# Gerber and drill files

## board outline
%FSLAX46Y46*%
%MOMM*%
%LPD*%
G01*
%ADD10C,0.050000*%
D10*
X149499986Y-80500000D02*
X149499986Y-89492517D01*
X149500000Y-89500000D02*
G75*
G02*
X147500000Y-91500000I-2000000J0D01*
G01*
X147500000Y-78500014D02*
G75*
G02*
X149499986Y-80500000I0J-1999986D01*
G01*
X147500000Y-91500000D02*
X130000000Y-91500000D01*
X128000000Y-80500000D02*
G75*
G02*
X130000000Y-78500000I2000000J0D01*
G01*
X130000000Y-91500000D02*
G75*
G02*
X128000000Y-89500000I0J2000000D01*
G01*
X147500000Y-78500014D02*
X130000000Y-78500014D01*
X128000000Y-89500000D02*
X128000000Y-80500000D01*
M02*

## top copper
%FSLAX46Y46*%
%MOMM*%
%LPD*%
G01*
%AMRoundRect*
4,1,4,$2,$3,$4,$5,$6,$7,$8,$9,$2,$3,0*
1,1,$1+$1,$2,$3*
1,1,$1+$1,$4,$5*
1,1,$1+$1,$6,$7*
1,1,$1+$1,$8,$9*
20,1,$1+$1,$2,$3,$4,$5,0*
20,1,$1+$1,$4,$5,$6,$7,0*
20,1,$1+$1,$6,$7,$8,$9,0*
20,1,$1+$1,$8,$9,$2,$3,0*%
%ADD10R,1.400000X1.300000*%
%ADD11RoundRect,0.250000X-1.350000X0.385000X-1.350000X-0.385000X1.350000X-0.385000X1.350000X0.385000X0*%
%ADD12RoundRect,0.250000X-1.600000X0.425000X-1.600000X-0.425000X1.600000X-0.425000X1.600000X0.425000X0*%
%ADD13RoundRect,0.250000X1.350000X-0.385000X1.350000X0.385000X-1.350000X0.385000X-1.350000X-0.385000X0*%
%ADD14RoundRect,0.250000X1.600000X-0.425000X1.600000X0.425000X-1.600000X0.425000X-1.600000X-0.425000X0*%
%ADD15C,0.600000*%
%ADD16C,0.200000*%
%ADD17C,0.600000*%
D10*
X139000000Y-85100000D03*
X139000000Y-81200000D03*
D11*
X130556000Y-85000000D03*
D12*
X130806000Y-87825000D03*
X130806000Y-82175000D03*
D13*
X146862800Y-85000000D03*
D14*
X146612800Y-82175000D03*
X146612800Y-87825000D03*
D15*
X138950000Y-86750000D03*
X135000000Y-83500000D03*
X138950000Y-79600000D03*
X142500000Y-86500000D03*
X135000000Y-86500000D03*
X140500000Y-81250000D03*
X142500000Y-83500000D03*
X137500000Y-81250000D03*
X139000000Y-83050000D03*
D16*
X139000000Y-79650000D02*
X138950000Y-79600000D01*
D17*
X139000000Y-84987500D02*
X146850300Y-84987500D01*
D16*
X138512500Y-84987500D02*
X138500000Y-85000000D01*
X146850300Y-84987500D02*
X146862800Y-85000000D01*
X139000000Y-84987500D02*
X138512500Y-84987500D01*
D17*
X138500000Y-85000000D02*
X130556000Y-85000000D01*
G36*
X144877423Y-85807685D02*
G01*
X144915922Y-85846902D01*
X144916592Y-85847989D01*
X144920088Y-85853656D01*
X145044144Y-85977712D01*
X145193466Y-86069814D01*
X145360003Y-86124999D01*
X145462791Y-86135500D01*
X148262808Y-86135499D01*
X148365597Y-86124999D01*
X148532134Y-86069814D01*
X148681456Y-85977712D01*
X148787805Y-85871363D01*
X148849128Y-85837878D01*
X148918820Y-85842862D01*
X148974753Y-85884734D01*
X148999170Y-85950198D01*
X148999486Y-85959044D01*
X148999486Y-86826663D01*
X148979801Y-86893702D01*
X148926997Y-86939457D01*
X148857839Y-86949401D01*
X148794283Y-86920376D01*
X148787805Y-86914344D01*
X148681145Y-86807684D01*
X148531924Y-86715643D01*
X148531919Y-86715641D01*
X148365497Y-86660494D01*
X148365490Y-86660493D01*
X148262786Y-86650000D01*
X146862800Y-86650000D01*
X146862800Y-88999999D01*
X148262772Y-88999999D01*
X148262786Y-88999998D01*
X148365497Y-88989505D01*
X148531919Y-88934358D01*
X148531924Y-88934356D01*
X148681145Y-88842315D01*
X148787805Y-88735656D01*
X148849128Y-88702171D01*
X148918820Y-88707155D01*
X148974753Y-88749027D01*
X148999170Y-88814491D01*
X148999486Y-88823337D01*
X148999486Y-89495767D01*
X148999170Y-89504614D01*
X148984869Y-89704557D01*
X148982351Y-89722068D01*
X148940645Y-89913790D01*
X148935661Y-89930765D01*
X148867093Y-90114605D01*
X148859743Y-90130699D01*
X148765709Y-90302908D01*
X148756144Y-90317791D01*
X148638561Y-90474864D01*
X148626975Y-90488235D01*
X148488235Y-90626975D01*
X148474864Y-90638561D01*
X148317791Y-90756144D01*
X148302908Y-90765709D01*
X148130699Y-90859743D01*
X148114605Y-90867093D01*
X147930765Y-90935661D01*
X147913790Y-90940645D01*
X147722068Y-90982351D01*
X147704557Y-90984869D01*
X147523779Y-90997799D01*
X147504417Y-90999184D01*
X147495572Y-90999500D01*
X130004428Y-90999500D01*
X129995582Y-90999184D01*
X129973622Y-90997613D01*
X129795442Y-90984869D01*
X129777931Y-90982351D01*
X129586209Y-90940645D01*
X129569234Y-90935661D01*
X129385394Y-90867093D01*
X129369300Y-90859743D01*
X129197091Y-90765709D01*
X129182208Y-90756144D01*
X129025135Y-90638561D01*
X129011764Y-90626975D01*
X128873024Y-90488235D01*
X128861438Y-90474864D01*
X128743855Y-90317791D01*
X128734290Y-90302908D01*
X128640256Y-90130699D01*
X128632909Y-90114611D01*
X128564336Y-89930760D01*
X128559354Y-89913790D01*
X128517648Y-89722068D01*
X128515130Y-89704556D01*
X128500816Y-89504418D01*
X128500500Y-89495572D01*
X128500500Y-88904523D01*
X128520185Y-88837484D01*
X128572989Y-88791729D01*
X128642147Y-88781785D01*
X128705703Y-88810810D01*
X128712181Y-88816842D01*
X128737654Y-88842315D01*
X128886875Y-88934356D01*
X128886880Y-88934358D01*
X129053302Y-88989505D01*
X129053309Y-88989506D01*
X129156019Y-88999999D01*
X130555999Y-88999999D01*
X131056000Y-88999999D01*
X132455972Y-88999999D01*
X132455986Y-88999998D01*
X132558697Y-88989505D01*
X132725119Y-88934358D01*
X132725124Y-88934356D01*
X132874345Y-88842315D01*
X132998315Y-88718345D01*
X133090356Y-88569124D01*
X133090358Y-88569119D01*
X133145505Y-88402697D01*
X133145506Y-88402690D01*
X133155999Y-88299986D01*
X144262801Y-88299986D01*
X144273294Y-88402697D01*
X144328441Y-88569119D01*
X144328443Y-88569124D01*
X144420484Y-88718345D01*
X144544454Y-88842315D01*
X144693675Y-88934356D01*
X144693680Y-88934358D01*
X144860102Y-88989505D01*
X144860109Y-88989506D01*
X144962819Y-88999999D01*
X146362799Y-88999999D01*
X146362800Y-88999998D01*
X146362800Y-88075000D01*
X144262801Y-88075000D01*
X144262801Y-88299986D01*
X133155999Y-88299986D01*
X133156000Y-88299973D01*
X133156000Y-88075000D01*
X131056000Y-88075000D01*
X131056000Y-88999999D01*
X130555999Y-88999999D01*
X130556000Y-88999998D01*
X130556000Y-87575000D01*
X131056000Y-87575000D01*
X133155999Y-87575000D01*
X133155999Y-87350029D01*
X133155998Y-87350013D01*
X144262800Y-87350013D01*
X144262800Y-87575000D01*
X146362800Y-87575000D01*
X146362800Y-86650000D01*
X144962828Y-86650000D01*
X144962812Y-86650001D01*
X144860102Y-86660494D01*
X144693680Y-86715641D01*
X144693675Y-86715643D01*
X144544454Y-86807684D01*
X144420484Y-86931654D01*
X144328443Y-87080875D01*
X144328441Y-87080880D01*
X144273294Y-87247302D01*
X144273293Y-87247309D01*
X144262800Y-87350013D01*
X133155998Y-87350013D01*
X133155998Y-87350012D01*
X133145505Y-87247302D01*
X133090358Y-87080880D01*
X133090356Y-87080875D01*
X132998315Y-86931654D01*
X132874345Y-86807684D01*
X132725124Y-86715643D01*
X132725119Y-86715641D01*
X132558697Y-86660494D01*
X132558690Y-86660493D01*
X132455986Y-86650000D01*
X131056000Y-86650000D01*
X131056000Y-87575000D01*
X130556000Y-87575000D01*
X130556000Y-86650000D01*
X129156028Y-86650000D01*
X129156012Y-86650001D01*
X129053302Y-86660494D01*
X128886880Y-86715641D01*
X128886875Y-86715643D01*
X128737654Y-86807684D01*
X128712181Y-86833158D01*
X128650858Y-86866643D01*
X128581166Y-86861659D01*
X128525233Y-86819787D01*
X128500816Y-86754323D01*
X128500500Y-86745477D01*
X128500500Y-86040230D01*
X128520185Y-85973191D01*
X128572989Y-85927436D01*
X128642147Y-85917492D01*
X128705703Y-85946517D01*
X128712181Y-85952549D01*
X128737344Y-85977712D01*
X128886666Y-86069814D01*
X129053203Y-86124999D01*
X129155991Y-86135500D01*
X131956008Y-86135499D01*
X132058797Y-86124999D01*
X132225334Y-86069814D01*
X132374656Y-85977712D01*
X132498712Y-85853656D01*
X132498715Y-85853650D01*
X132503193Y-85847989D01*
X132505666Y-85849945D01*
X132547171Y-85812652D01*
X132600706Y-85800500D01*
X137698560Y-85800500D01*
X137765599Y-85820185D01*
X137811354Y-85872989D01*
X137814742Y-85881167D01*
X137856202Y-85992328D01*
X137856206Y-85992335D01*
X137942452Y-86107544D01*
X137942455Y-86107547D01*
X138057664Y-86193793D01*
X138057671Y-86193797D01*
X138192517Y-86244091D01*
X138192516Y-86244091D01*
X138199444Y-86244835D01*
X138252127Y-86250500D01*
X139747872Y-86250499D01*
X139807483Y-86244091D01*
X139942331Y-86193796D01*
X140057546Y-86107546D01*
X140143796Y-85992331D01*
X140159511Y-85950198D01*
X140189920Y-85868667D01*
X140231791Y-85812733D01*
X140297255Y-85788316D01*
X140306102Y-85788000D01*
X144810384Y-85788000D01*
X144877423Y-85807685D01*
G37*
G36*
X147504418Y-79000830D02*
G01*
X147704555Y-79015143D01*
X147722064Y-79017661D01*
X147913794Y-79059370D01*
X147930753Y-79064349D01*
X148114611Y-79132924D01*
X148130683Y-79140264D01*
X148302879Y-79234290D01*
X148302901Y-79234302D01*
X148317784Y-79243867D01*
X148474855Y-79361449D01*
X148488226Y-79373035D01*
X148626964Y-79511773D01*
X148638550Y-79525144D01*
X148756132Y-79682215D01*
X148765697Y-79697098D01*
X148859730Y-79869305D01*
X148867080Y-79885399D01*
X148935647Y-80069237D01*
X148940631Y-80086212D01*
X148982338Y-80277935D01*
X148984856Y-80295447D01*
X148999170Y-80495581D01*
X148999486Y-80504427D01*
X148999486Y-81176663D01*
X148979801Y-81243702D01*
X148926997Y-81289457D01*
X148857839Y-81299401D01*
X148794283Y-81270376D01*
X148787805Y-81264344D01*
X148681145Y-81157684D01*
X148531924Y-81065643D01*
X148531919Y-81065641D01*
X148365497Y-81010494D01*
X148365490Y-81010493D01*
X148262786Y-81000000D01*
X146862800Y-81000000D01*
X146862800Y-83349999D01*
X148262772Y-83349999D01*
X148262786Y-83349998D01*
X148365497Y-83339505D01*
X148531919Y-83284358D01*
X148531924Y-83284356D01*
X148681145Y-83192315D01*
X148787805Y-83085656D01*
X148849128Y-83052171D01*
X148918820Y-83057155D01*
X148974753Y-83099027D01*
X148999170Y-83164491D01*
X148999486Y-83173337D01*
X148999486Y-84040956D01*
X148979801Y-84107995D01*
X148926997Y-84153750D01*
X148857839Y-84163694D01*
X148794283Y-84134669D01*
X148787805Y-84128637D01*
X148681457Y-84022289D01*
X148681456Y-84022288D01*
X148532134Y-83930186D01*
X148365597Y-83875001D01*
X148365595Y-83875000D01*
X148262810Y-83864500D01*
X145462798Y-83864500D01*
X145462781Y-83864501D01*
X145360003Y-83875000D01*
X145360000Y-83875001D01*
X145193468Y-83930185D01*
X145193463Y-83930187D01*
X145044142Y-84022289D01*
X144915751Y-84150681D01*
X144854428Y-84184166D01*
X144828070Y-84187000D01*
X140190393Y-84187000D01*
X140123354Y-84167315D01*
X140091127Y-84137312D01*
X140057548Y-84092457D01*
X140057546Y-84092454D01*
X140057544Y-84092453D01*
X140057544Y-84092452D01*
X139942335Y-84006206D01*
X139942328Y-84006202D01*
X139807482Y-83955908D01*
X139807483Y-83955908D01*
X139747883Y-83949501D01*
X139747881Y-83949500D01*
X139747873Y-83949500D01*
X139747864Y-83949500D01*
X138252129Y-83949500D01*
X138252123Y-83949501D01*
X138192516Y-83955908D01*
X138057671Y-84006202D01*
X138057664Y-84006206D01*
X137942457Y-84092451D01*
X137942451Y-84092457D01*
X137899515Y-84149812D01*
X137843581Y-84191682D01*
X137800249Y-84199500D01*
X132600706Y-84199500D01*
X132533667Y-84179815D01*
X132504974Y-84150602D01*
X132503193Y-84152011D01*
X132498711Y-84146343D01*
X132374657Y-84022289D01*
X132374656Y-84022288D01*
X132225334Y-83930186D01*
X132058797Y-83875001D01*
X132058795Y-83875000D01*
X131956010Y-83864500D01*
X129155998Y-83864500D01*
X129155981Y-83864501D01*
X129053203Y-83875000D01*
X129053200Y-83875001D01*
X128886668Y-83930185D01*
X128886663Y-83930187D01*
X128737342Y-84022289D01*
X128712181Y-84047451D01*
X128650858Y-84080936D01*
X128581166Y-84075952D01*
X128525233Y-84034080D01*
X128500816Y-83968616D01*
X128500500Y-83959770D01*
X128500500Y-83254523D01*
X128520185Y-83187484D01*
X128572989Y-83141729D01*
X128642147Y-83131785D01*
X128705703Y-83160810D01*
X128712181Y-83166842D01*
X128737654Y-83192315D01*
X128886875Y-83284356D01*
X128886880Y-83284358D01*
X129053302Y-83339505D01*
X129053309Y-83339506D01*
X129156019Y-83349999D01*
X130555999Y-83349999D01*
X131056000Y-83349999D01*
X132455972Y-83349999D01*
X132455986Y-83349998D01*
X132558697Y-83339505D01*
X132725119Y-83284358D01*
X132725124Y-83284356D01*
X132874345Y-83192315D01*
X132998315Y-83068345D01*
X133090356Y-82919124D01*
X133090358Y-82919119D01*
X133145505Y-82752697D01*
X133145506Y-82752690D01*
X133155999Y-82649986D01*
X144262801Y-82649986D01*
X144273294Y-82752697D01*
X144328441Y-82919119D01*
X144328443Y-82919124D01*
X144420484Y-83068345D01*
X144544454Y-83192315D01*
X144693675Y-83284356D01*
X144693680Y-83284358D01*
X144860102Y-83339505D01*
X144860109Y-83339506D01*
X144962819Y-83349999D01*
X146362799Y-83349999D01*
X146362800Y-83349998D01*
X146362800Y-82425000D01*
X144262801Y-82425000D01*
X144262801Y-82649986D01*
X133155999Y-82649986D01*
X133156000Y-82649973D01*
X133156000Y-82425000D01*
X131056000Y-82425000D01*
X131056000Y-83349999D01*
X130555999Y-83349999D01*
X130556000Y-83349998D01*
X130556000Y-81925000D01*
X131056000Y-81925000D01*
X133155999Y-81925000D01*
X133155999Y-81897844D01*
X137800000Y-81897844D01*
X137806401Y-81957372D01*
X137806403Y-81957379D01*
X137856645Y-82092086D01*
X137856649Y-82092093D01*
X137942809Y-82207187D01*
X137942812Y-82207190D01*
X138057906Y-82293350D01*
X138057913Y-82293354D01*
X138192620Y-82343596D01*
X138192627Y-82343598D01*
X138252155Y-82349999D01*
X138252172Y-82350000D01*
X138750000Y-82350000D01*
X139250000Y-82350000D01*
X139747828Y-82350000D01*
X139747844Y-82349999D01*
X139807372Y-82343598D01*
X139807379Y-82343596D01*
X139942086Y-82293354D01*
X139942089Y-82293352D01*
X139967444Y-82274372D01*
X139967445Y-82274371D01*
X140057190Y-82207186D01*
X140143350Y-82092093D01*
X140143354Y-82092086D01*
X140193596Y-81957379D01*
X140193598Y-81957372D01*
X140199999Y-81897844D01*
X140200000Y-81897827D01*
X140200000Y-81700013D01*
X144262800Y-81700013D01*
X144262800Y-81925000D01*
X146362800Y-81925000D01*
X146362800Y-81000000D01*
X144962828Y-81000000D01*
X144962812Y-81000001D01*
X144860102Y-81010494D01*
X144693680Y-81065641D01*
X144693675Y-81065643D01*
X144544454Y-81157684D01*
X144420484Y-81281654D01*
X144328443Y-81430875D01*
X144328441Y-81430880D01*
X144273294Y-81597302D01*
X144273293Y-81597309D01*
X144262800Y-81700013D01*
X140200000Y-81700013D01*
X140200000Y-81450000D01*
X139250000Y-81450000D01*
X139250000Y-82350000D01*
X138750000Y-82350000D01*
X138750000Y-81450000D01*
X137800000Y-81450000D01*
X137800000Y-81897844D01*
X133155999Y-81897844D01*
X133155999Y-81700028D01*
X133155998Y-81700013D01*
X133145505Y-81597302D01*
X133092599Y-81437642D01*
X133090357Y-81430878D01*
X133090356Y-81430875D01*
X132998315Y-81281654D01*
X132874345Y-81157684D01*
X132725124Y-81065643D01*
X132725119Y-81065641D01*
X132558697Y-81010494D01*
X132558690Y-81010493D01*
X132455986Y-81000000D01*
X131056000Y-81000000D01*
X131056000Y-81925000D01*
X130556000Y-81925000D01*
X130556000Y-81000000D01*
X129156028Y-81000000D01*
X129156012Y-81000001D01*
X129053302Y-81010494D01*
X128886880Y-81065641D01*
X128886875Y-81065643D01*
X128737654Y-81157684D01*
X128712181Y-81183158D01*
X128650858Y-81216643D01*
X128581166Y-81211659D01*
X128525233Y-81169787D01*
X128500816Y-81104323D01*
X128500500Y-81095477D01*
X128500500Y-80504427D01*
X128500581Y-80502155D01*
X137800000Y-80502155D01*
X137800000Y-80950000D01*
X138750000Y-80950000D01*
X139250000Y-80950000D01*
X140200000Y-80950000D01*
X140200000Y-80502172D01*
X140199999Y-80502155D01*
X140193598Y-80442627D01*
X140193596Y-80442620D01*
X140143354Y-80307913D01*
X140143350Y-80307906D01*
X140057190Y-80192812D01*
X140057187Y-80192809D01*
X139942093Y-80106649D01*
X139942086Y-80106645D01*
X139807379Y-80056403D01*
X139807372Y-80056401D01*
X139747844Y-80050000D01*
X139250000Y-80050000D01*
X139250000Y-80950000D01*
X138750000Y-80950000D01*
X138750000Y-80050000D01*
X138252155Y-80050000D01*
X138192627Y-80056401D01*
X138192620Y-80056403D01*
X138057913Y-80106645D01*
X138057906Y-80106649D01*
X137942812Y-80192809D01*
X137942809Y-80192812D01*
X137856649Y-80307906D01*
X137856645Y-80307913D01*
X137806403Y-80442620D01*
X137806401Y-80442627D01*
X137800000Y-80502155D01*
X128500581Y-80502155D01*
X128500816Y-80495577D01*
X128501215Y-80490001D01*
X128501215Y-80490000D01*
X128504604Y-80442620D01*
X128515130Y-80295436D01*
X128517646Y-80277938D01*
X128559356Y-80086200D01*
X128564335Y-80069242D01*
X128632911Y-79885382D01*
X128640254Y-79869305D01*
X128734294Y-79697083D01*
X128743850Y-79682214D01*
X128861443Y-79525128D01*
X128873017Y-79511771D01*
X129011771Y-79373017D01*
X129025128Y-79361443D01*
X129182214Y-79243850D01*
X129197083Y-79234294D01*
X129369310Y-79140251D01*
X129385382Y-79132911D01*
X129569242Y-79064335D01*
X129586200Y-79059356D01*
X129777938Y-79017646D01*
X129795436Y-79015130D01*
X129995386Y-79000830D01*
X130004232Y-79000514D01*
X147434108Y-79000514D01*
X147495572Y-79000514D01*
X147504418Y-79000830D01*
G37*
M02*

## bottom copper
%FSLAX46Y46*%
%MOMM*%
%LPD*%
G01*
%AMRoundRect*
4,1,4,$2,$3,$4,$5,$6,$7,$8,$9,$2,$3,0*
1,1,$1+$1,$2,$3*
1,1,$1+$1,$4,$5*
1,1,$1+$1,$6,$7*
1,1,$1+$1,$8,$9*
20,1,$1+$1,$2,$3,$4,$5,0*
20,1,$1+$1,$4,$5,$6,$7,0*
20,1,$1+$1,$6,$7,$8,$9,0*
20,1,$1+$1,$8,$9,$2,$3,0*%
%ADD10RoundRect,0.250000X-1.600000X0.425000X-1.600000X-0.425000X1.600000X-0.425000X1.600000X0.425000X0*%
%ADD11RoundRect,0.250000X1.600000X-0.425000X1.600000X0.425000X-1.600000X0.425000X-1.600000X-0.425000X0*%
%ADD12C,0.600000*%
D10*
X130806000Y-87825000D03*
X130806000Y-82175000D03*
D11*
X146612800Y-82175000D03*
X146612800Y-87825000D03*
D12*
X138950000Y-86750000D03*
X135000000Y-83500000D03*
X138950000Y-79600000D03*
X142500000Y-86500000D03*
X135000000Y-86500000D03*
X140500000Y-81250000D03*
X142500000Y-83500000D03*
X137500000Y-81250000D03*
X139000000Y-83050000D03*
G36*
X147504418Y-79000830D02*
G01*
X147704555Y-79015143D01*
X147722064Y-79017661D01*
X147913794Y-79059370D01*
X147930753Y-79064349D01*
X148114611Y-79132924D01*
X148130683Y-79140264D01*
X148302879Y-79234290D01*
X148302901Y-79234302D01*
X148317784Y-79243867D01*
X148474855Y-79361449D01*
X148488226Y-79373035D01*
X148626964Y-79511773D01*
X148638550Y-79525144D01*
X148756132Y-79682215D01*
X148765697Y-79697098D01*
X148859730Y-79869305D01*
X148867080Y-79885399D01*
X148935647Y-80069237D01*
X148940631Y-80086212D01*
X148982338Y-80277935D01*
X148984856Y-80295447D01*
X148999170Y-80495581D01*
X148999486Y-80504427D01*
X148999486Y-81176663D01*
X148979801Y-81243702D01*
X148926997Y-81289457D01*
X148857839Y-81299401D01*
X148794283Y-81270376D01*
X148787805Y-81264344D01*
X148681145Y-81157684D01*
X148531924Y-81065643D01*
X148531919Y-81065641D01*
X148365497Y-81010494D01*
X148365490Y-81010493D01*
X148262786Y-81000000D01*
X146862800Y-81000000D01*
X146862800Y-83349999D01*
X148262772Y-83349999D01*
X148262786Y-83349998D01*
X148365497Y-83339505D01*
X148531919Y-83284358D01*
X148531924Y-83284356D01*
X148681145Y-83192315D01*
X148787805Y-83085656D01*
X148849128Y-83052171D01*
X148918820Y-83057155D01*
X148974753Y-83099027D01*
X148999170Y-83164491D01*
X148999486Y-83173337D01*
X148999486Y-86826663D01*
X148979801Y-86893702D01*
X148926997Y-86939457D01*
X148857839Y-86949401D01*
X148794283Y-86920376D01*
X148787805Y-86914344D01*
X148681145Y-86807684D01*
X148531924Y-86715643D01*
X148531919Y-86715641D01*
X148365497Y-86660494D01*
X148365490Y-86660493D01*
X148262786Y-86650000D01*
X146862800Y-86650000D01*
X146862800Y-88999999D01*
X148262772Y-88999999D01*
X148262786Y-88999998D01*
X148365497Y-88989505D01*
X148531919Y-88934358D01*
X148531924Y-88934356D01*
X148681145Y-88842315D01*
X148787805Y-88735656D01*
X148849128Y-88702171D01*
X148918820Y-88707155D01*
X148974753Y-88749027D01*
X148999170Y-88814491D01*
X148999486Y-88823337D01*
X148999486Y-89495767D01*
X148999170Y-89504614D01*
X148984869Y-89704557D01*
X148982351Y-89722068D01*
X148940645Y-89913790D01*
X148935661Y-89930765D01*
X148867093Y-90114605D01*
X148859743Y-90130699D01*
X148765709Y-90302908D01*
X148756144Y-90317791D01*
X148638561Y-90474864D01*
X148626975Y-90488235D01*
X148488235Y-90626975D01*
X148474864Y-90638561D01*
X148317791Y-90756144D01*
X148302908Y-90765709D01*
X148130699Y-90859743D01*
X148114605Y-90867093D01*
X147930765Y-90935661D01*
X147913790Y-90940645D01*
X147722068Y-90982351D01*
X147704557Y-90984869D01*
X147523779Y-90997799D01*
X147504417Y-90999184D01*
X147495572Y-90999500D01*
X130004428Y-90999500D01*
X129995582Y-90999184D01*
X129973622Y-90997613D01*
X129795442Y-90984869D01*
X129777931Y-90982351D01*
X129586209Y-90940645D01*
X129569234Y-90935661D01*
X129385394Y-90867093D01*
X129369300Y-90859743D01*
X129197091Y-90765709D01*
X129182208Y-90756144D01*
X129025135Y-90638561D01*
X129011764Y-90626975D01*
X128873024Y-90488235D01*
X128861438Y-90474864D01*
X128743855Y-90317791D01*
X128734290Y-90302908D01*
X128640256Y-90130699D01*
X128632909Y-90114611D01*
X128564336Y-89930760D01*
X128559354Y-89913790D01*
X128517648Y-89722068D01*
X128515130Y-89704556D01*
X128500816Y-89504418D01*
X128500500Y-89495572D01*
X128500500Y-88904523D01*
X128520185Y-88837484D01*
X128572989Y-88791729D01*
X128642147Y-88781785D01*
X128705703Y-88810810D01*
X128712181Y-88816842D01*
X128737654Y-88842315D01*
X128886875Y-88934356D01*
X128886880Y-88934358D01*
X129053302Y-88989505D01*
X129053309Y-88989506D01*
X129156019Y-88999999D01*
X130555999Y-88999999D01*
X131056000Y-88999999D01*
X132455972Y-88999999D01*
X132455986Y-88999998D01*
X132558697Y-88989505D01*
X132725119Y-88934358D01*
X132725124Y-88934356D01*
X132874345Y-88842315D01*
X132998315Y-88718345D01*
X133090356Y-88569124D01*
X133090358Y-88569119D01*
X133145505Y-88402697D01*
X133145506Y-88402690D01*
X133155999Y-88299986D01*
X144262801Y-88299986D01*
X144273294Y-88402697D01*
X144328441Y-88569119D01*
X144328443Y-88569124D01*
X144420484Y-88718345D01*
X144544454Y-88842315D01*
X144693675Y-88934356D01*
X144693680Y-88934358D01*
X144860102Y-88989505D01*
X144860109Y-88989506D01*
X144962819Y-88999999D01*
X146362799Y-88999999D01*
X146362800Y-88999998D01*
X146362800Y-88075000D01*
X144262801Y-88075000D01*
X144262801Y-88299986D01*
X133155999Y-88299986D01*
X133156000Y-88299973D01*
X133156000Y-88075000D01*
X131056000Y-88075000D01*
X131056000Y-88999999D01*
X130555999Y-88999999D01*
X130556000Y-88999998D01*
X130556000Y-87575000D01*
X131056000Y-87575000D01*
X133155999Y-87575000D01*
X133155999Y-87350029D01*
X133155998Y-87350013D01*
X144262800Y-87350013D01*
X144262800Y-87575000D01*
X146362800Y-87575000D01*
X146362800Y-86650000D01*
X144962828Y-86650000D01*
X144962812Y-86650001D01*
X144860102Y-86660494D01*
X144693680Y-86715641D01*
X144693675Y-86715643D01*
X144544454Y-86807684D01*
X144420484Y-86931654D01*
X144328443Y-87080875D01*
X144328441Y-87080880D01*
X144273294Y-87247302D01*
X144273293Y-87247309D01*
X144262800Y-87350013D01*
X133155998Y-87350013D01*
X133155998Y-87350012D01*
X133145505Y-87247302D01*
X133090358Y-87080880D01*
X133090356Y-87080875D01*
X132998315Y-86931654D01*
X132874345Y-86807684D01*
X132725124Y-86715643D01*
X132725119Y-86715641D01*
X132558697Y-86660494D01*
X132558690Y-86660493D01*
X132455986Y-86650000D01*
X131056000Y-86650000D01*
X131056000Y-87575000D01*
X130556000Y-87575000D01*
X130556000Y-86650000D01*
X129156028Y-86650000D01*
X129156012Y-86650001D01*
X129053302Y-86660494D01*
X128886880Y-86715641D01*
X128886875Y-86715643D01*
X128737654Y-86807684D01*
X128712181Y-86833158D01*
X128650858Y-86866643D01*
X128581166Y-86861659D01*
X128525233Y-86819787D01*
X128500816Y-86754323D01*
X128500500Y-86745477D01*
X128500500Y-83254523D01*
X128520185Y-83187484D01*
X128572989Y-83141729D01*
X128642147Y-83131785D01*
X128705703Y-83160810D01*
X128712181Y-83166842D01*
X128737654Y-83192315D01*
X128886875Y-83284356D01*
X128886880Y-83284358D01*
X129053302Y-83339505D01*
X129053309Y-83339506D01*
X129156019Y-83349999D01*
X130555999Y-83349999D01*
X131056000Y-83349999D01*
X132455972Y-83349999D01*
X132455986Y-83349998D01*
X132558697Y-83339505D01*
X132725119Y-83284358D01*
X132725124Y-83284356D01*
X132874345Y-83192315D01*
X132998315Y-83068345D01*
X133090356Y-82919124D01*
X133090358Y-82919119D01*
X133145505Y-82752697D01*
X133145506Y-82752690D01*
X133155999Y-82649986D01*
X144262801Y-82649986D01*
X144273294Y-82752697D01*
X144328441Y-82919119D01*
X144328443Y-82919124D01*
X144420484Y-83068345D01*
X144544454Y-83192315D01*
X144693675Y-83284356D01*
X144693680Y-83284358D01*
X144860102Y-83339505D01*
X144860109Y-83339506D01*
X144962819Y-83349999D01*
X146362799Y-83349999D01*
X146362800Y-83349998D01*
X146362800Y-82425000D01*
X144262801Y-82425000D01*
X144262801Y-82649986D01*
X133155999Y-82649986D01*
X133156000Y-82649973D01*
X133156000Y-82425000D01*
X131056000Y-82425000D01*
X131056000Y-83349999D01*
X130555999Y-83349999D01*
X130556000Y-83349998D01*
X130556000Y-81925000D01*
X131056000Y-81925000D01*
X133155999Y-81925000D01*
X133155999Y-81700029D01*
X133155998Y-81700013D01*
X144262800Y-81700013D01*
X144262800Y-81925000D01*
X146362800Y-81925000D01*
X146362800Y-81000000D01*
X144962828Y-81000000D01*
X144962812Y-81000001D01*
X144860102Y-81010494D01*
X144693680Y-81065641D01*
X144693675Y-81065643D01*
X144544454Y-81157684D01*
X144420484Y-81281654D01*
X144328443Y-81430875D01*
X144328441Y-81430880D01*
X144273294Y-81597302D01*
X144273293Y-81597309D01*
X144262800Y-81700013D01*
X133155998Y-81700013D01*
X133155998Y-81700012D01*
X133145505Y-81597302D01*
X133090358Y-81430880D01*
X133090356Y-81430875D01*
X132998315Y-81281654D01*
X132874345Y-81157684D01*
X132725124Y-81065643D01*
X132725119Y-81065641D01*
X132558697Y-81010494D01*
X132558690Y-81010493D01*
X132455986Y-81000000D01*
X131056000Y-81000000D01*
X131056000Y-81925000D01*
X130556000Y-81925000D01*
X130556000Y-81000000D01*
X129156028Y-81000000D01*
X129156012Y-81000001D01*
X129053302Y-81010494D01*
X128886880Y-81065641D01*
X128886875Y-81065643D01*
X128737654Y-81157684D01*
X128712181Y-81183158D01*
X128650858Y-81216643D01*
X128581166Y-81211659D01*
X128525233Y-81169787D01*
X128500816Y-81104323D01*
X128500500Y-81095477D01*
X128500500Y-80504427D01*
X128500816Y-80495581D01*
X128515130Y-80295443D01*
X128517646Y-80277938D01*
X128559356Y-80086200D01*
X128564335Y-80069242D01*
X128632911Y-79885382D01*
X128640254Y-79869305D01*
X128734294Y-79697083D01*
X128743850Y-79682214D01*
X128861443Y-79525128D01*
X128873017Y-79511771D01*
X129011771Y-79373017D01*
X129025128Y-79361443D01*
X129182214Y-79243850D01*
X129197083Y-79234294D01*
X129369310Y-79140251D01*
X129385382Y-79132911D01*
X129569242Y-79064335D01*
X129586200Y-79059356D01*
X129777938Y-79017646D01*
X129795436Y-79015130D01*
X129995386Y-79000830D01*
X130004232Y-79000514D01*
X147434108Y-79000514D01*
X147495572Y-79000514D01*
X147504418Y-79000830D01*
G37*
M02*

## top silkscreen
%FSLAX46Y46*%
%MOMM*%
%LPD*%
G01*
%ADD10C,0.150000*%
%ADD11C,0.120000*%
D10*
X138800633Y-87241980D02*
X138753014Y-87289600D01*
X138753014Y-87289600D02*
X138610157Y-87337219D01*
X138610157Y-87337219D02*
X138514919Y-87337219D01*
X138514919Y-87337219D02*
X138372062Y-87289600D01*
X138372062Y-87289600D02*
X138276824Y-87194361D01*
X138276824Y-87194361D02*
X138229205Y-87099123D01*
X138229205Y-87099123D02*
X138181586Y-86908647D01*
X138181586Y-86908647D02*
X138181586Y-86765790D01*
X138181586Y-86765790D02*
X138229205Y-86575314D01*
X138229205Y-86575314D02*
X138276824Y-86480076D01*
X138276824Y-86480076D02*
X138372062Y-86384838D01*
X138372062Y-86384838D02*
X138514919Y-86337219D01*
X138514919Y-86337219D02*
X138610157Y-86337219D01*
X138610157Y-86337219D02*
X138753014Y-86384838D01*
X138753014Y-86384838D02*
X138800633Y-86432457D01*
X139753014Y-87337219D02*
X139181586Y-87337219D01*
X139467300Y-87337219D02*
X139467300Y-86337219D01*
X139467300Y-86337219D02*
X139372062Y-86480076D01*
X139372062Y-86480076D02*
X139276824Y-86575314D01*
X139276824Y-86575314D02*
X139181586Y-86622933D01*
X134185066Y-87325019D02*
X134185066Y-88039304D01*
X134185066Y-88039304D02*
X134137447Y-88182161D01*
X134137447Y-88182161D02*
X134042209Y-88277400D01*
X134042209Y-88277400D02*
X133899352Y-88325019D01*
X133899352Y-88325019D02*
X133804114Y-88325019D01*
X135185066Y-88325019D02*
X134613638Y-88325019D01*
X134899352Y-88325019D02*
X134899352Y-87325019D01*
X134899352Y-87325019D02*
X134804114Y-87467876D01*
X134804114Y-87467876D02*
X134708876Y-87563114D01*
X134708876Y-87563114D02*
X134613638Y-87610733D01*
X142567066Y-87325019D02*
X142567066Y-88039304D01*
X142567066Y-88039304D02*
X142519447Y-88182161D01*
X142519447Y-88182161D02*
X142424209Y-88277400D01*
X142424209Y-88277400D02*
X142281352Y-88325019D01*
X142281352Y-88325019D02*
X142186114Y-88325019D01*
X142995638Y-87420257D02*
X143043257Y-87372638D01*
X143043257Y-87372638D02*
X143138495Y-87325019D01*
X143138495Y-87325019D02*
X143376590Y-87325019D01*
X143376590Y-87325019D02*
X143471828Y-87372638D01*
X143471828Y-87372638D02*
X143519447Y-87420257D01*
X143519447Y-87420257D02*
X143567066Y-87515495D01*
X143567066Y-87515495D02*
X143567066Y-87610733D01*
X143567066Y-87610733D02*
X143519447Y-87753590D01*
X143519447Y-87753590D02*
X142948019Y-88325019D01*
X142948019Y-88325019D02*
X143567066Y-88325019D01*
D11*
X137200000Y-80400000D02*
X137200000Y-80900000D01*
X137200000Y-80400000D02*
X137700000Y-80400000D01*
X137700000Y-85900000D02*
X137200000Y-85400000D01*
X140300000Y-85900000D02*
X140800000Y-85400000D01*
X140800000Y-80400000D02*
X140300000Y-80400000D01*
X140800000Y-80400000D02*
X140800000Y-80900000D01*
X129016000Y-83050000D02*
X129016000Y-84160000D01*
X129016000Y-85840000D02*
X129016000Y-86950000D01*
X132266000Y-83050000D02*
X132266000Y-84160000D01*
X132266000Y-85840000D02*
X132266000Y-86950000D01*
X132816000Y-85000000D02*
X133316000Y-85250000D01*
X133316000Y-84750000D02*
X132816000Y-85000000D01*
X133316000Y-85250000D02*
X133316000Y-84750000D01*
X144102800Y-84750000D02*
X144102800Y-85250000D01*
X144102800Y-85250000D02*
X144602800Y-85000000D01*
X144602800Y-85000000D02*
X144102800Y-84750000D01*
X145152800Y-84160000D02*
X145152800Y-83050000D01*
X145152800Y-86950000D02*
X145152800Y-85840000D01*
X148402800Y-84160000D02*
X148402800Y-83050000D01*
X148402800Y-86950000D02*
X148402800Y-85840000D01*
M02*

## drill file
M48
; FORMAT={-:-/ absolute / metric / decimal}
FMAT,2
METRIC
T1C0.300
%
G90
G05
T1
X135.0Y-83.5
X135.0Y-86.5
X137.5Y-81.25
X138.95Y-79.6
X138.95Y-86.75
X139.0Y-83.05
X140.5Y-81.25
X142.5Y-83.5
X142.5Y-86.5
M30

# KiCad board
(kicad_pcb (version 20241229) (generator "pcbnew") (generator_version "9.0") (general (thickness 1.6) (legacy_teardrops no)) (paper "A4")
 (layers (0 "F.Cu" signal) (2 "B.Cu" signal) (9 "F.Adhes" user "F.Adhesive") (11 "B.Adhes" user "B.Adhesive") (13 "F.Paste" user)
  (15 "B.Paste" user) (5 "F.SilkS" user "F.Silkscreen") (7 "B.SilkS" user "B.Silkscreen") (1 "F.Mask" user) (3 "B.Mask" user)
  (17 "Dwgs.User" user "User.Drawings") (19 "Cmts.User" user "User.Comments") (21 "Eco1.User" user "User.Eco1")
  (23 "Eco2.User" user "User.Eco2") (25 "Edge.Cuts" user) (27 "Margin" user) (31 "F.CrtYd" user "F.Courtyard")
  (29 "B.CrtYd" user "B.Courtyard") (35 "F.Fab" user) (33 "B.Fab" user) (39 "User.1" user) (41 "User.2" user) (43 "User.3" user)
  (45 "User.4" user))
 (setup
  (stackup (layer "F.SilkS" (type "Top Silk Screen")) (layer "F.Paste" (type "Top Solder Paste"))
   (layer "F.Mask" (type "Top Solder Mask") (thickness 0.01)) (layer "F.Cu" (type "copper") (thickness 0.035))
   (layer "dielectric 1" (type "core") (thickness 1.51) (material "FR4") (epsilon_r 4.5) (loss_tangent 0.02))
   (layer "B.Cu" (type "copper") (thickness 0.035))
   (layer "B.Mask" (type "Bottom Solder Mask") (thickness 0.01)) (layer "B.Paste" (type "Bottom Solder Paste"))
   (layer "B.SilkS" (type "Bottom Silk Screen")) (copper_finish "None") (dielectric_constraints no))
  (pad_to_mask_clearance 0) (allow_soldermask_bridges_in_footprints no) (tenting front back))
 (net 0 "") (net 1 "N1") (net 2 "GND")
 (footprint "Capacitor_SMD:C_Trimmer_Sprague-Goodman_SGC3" (layer "F.Cu") (at 139 83.15 90)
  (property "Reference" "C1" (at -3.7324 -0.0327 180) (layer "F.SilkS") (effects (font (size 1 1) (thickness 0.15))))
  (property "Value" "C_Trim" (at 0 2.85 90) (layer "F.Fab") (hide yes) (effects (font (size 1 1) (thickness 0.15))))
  (fp_line (start 2.75 -1.8) (end 2.25 -1.8) (stroke (width 0.12) (type solid)) (layer "F.SilkS"))
  (fp_line (start 2.75 -1.8) (end 2.75 -1.3) (stroke (width 0.12) (type solid)) (layer "F.SilkS"))
  (fp_line (start -2.75 -1.3) (end -2.25 -1.8) (stroke (width 0.12) (type solid)) (layer "F.SilkS"))
  (fp_line (start -2.75 1.3) (end -2.25 1.8) (stroke (width 0.12) (type solid)) (layer "F.SilkS"))
  (fp_line (start 2.75 1.8) (end 2.75 1.3) (stroke (width 0.12) (type solid)) (layer "F.SilkS"))
  (fp_line (start 2.75 1.8) (end 2.25 1.8) (stroke (width 0.12) (type solid)) (layer "F.SilkS"))
  (pad "1" smd rect (at -1.95 0 90) (size 1.3 1.4) (layers "F.Cu" "F.Mask" "F.Paste") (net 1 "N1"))
  (pad "2" smd rect (at 1.95 0 90) (size 1.3 1.4) (layers "F.Cu" "F.Mask" "F.Paste") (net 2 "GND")))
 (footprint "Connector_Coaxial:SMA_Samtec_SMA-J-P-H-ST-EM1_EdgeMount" (layer "F.Cu") (at 130.556 85 180)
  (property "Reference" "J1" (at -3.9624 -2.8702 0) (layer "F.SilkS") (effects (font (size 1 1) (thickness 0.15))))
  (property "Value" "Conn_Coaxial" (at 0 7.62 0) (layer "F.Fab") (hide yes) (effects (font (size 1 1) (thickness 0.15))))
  (fp_line (start 1.54 1.95) (end 1.54 0.84) (stroke (width 0.12) (type solid)) (layer "F.SilkS"))
  (fp_line (start 1.54 -0.84) (end 1.54 -1.95) (stroke (width 0.12) (type solid)) (layer "F.SilkS"))
  (fp_line (start -1.71 1.95) (end -1.71 0.84) (stroke (width 0.12) (type solid)) (layer "F.SilkS"))
  (fp_line (start -1.71 -0.84) (end -1.71 -1.95) (stroke (width 0.12) (type solid)) (layer "F.SilkS"))
  (fp_line (start -2.26 0) (end -2.76 -0.25) (stroke (width 0.12) (type solid)) (layer "F.SilkS"))
  (fp_line (start -2.76 0.25) (end -2.26 0) (stroke (width 0.12) (type solid)) (layer "F.SilkS"))
  (fp_line (start -2.76 -0.25) (end -2.76 0.25) (stroke (width 0.12) (type solid)) (layer "F.SilkS"))
  (pad "1" smd roundrect (at 0 0 270) (size 1.27 3.2) (layers "F.Cu" "F.Mask") (roundrect_rratio 0.1968503937) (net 1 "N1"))
  (pad "2" smd roundrect (at -0.25 -2.825 270) (size 1.35 3.7) (layers "F.Cu" "F.Mask") (roundrect_rratio 0.1851851852) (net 2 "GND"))
  (pad "2" smd roundrect (at -0.25 -2.825 270) (size 1.35 3.7) (layers "B.Cu" "B.Mask") (roundrect_rratio 0.1851851852) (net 2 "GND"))
  (pad "2" smd roundrect (at -0.25 2.825 270) (size 1.35 3.7) (layers "F.Cu" "F.Mask") (roundrect_rratio 0.1851851852) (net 2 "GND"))
  (pad "2" smd roundrect (at -0.25 2.825 270) (size 1.35 3.7) (layers "B.Cu" "B.Mask") (roundrect_rratio 0.1851851852) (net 2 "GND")))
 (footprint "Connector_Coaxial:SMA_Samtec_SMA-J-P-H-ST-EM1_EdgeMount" (layer "F.Cu") (at 146.8628 85)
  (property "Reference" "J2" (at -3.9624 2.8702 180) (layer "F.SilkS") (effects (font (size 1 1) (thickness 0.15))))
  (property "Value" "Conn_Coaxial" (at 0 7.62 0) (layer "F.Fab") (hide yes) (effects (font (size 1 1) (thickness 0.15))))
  (fp_line (start -2.76 -0.25) (end -2.76 0.25) (stroke (width 0.12) (type solid)) (layer "F.SilkS"))
  (fp_line (start -2.76 0.25) (end -2.26 0) (stroke (width 0.12) (type solid)) (layer "F.SilkS"))
  (fp_line (start -2.26 0) (end -2.76 -0.25) (stroke (width 0.12) (type solid)) (layer "F.SilkS"))
  (fp_line (start -1.71 -0.84) (end -1.71 -1.95) (stroke (width 0.12) (type solid)) (layer "F.SilkS"))
  (fp_line (start -1.71 1.95) (end -1.71 0.84) (stroke (width 0.12) (type solid)) (layer "F.SilkS"))
  (fp_line (start 1.54 -0.84) (end 1.54 -1.95) (stroke (width 0.12) (type solid)) (layer "F.SilkS"))
  (fp_line (start 1.54 1.95) (end 1.54 0.84) (stroke (width 0.12) (type solid)) (layer "F.SilkS"))
  (pad "1" smd roundrect (at 0 0 90) (size 1.27 3.2) (layers "F.Cu" "F.Mask") (roundrect_rratio 0.1968503937) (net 1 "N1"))
  (pad "2" smd roundrect (at -0.25 -2.825 90) (size 1.35 3.7) (layers "F.Cu" "F.Mask") (roundrect_rratio 0.1851851852) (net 2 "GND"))
  (pad "2" smd roundrect (at -0.25 -2.825 90) (size 1.35 3.7) (layers "B.Cu" "B.Mask") (roundrect_rratio 0.1851851852) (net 2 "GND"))
  (pad "2" smd roundrect (at -0.25 2.825 90) (size 1.35 3.7) (layers "F.Cu" "F.Mask") (roundrect_rratio 0.1851851852) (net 2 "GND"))
  (pad "2" smd roundrect (at -0.25 2.825 90) (size 1.35 3.7) (layers "B.Cu" "B.Mask") (roundrect_rratio 0.1851851852) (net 2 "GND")))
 (gr_line (start 149.499986 80.5) (end 149.499986 89.492517) (stroke (width 0.05) (type default)) (layer "Edge.Cuts"))
 (gr_arc (start 149.5 89.5) (mid 148.914214 90.914214) (end 147.5 91.5) (stroke (width 0.05) (type solid)) (layer "Edge.Cuts"))
 (gr_arc (start 147.5 78.500014) (mid 148.914204 79.085796) (end 149.499986 80.5) (stroke (width 0.05) (type default)) (layer "Edge.Cuts"))
 (gr_line (start 147.5 91.5) (end 130 91.5) (stroke (width 0.05) (type default)) (layer "Edge.Cuts"))
 (gr_arc (start 128 80.5) (mid 128.585786 79.085786) (end 130 78.5) (stroke (width 0.05) (type solid)) (layer "Edge.Cuts"))
 (gr_arc (start 130 91.5) (mid 128.585786 90.914214) (end 128 89.5) (stroke (width 0.05) (type default)) (layer "Edge.Cuts"))
 (gr_line (start 147.5 78.500014) (end 130 78.500014) (stroke (width 0.05) (type default)) (layer "Edge.Cuts"))
 (gr_line (start 128 89.5) (end 128 80.5) (stroke (width 0.05) (type default)) (layer "Edge.Cuts"))
 (segment (start 139 79.65) (end 138.95 79.6) (width 0.2) (layer "F.Cu") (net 2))
 (via (at 138.95 86.75) (size 0.6) (drill 0.3) (layers "F.Cu" "B.Cu") (free yes) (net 2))
 (via (at 135 83.5) (size 0.6) (drill 0.3) (layers "F.Cu" "B.Cu") (free yes) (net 2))
 (via (at 138.95 79.6) (size 0.6) (drill 0.3) (layers "F.Cu" "B.Cu") (free yes) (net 2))
 (via (at 142.5 86.5) (size 0.6) (drill 0.3) (layers "F.Cu" "B.Cu") (free yes) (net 2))
 (via (at 135 86.5) (size 0.6) (drill 0.3) (layers "F.Cu" "B.Cu") (free yes) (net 2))
 (via (at 140.5 81.25) (size 0.6) (drill 0.3) (layers "F.Cu" "B.Cu") (free yes) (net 2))
 (via (at 142.5 83.5) (size 0.6) (drill 0.3) (layers "F.Cu" "B.Cu") (free yes) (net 2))
 (via (at 137.5 81.25) (size 0.6) (drill 0.3) (layers "F.Cu" "B.Cu") (free yes) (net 2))
 (via (at 139 83.05) (size 0.6) (drill 0.3) (layers "F.Cu" "B.Cu") (free yes) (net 2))
 (segment (start 139 84.9875) (end 146.8503 84.9875) (width 0.6) (layer "F.Cu") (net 1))
 (segment (start 138.5125 84.9875) (end 138.5 85) (width 0.2) (layer "F.Cu") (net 1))
 (segment (start 146.8503 84.9875) (end 146.8628 85) (width 0.2) (layer "F.Cu") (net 1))
 (segment (start 139 84.9875) (end 138.5125 84.9875) (width 0.2) (layer "F.Cu") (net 1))
 (segment (start 138.5 85) (end 130.556 85) (width 0.6) (layer "F.Cu") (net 1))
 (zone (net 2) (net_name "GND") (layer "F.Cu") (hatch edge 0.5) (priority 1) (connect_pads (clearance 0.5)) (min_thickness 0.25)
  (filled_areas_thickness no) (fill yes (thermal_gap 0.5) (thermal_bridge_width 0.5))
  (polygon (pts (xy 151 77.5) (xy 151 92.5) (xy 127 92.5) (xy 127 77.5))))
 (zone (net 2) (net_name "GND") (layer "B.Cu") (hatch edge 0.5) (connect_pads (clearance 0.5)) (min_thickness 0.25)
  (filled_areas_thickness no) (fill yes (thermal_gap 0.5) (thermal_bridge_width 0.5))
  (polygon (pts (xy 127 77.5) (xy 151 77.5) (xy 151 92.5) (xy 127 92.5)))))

